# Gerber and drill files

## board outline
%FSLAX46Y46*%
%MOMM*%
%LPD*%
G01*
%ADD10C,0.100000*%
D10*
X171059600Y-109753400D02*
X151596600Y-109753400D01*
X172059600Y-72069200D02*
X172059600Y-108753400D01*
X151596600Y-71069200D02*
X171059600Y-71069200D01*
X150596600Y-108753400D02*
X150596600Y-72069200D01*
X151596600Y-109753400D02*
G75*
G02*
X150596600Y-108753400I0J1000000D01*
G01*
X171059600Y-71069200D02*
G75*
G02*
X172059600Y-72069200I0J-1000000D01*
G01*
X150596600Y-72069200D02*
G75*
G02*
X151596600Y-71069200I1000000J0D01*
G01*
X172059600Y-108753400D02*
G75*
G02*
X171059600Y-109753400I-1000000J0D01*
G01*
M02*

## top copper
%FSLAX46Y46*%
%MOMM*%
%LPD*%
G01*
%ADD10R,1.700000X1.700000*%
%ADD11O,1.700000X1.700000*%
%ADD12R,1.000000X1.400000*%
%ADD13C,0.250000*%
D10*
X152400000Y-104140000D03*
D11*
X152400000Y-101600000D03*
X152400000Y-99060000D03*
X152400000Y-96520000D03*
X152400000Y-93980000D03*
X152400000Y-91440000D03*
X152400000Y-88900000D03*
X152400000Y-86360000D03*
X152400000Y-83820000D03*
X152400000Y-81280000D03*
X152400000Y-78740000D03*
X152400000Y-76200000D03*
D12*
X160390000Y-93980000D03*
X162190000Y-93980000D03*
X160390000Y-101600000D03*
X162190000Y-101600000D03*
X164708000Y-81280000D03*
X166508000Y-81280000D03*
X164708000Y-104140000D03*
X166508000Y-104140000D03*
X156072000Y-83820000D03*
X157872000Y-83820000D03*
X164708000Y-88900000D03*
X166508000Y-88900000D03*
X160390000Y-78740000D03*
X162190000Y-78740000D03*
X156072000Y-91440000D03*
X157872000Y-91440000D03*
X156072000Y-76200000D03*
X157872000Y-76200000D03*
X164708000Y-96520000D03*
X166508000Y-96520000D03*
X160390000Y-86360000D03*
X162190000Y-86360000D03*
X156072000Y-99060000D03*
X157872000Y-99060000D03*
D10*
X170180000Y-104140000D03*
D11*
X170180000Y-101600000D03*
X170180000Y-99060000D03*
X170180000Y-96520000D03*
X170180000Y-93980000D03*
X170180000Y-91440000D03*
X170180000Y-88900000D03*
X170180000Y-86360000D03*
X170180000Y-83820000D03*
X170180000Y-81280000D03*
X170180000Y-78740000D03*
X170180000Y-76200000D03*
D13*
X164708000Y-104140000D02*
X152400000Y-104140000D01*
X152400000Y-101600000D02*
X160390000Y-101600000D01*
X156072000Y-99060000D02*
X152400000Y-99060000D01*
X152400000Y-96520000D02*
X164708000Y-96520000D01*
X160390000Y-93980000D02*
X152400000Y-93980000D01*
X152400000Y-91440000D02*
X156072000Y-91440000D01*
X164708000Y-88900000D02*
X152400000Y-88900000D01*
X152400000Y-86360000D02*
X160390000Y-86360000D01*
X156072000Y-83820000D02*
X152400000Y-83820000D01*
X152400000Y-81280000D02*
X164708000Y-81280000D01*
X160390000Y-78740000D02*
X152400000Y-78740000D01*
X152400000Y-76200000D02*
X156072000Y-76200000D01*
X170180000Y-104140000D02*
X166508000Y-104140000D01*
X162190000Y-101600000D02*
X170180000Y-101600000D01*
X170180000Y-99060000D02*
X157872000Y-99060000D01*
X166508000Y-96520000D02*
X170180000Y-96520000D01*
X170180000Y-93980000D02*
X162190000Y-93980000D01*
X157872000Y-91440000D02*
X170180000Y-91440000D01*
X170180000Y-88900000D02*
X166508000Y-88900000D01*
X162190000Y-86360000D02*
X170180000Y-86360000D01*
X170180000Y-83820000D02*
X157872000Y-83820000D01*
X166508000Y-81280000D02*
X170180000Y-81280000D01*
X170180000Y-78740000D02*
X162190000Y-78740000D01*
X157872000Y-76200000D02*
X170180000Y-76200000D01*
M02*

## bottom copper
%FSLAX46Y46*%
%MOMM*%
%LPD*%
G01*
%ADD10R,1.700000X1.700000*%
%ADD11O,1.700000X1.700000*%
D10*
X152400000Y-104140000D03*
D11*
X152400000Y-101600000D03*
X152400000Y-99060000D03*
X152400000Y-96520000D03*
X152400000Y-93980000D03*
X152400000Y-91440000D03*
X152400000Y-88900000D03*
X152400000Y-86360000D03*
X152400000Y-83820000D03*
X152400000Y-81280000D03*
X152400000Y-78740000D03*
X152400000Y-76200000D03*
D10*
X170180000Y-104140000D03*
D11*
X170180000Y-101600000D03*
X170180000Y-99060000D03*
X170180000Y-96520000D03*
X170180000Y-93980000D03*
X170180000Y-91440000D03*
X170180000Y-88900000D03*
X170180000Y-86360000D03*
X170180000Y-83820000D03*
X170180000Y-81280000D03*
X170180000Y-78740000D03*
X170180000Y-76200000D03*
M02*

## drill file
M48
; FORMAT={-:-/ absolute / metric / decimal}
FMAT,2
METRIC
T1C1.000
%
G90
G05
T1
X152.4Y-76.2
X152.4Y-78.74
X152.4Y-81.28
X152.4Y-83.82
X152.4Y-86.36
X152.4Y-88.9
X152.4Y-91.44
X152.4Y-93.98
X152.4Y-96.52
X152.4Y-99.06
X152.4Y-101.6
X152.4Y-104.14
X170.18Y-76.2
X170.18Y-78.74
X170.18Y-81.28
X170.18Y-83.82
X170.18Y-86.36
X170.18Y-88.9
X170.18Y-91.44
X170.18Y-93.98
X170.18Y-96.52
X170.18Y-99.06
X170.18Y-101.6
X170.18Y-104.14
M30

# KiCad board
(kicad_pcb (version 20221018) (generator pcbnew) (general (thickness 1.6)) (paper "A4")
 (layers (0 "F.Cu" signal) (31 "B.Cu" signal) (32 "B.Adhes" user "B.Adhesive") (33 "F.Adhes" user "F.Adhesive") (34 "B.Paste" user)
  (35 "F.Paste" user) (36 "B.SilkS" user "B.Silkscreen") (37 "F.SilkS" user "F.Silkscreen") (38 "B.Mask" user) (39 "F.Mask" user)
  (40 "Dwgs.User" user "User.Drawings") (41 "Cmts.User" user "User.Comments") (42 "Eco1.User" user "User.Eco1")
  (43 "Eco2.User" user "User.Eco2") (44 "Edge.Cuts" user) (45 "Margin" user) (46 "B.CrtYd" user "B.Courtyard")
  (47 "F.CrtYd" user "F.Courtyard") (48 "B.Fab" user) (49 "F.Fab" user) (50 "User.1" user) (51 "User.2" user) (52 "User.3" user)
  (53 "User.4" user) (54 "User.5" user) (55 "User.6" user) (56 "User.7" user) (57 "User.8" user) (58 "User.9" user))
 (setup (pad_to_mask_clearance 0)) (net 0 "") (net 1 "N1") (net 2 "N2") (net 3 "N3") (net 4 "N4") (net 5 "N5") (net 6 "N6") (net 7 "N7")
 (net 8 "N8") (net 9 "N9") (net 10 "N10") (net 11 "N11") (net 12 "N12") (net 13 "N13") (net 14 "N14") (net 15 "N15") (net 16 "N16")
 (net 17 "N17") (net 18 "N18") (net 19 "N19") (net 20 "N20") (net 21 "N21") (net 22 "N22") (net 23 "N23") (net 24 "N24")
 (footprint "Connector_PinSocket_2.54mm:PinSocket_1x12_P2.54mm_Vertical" (layer "F.Cu") (at 152.4 104.14 180)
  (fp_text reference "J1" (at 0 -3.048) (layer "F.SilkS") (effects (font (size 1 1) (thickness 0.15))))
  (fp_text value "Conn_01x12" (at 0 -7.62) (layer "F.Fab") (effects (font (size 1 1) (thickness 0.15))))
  (pad "1" thru_hole rect (at 0 0 180) (size 1.7 1.7) (drill 1) (layers "*.Cu" "*.Mask") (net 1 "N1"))
  (pad "2" thru_hole oval (at 0 2.54 180) (size 1.7 1.7) (drill 1) (layers "*.Cu" "*.Mask") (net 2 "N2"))
  (pad "3" thru_hole oval (at 0 5.08 180) (size 1.7 1.7) (drill 1) (layers "*.Cu" "*.Mask") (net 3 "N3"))
  (pad "4" thru_hole oval (at 0 7.62 180) (size 1.7 1.7) (drill 1) (layers "*.Cu" "*.Mask") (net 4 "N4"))
  (pad "5" thru_hole oval (at 0 10.16 180) (size 1.7 1.7) (drill 1) (layers "*.Cu" "*.Mask") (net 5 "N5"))
  (pad "6" thru_hole oval (at 0 12.7 180) (size 1.7 1.7) (drill 1) (layers "*.Cu" "*.Mask") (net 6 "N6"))
  (pad "7" thru_hole oval (at 0 15.24 180) (size 1.7 1.7) (drill 1) (layers "*.Cu" "*.Mask") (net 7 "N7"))
  (pad "8" thru_hole oval (at 0 17.78 180) (size 1.7 1.7) (drill 1) (layers "*.Cu" "*.Mask") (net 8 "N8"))
  (pad "9" thru_hole oval (at 0 20.32 180) (size 1.7 1.7) (drill 1) (layers "*.Cu" "*.Mask") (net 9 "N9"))
  (pad "10" thru_hole oval (at 0 22.86 180) (size 1.7 1.7) (drill 1) (layers "*.Cu" "*.Mask") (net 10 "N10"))
  (pad "11" thru_hole oval (at 0 25.4 180) (size 1.7 1.7) (drill 1) (layers "*.Cu" "*.Mask") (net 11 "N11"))
  (pad "12" thru_hole oval (at 0 27.94 180) (size 1.7 1.7) (drill 1) (layers "*.Cu" "*.Mask") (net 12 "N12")))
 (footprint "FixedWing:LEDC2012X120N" (layer "F.Cu") (at 161.29 93.98)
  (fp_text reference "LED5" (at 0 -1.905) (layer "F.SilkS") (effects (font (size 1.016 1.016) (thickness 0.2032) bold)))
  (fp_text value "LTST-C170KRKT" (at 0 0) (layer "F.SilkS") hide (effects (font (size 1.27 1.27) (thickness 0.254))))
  (pad "1" smd rect (at -0.9 0) (size 1 1.4) (layers "F.Cu" "F.Paste" "F.Mask") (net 5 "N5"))
  (pad "2" smd rect (at 0.9 0) (size 1 1.4) (layers "F.Cu" "F.Paste" "F.Mask") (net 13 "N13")))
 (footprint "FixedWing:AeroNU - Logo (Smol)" (layer "F.Cu") (at 157.380649 109.377388)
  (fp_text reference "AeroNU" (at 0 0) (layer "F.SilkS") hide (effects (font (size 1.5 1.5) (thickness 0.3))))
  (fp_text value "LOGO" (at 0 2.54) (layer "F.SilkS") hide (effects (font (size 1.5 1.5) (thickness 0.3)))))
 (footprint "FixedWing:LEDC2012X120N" (layer "F.Cu") (at 161.29 101.6)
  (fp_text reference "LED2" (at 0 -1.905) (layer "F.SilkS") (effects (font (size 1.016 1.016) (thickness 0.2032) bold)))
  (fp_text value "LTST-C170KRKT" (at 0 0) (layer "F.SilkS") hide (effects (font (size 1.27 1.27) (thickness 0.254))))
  (pad "1" smd rect (at -0.9 0) (size 1 1.4) (layers "F.Cu" "F.Paste" "F.Mask") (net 2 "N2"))
  (pad "2" smd rect (at 0.9 0) (size 1 1.4) (layers "F.Cu" "F.Paste" "F.Mask") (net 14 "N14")))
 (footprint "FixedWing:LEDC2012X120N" (layer "F.Cu") (at 165.608 81.28)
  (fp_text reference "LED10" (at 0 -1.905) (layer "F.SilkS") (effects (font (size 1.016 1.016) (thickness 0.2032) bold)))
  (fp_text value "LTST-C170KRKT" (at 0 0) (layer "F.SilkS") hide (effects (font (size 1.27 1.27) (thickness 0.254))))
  (pad "1" smd rect (at -0.9 0) (size 1 1.4) (layers "F.Cu" "F.Paste" "F.Mask") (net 10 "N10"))
  (pad "2" smd rect (at 0.9 0) (size 1 1.4) (layers "F.Cu" "F.Paste" "F.Mask") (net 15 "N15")))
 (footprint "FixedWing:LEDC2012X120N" (layer "F.Cu") (at 165.608 104.14)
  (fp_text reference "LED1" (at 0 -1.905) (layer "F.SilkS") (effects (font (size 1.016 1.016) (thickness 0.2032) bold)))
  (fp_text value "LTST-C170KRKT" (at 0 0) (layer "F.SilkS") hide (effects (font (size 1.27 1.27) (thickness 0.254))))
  (pad "1" smd rect (at -0.9 0) (size 1 1.4) (layers "F.Cu" "F.Paste" "F.Mask") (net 1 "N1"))
  (pad "2" smd rect (at 0.9 0) (size 1 1.4) (layers "F.Cu" "F.Paste" "F.Mask") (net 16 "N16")))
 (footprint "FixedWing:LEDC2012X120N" (layer "F.Cu") (at 156.972 83.82)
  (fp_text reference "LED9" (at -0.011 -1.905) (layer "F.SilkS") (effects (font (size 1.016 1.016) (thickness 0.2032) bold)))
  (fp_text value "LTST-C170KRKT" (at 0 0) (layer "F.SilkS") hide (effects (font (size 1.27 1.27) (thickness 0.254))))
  (pad "1" smd rect (at -0.9 0) (size 1 1.4) (layers "F.Cu" "F.Paste" "F.Mask") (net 9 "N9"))
  (pad "2" smd rect (at 0.9 0) (size 1 1.4) (layers "F.Cu" "F.Paste" "F.Mask") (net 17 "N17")))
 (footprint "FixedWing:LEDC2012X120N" (layer "F.Cu") (at 165.608 88.9)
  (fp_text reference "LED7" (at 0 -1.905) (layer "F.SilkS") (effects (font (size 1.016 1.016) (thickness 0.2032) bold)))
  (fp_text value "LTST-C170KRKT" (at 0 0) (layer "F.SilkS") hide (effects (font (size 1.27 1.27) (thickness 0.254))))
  (pad "1" smd rect (at -0.9 0) (size 1 1.4) (layers "F.Cu" "F.Paste" "F.Mask") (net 7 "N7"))
  (pad "2" smd rect (at 0.9 0) (size 1 1.4) (layers "F.Cu" "F.Paste" "F.Mask") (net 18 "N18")))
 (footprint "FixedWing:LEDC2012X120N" (layer "F.Cu") (at 161.29 78.74)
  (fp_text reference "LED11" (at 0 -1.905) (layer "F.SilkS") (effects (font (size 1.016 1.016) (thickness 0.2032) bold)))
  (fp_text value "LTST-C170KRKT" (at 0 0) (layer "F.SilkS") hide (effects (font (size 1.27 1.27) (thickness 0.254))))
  (pad "1" smd rect (at -0.9 0) (size 1 1.4) (layers "F.Cu" "F.Paste" "F.Mask") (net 11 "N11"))
  (pad "2" smd rect (at 0.9 0) (size 1 1.4) (layers "F.Cu" "F.Paste" "F.Mask") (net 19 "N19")))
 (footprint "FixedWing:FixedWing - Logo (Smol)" (layer "F.Cu") (at 165.3921 73.1774)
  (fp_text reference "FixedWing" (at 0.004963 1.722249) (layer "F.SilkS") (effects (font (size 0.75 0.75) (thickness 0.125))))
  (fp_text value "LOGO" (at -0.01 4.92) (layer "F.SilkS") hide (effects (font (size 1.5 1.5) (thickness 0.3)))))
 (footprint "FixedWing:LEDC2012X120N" (layer "F.Cu") (at 156.972 91.44)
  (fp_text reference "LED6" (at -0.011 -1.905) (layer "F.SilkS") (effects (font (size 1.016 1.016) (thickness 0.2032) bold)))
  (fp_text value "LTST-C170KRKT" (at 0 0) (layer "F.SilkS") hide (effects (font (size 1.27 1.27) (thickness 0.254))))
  (pad "1" smd rect (at -0.9 0) (size 1 1.4) (layers "F.Cu" "F.Paste" "F.Mask") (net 6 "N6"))
  (pad "2" smd rect (at 0.9 0) (size 1 1.4) (layers "F.Cu" "F.Paste" "F.Mask") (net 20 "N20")))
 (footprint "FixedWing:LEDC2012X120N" (layer "F.Cu") (at 156.972 76.2)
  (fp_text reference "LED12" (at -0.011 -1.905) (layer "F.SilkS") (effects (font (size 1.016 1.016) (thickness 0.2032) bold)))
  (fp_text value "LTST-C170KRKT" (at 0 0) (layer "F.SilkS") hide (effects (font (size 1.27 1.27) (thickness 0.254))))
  (pad "1" smd rect (at -0.9 0) (size 1 1.4) (layers "F.Cu" "F.Paste" "F.Mask") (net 12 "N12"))
  (pad "2" smd rect (at 0.9 0) (size 1 1.4) (layers "F.Cu" "F.Paste" "F.Mask") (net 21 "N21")))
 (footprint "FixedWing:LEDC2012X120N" (layer "F.Cu") (at 165.608 96.52)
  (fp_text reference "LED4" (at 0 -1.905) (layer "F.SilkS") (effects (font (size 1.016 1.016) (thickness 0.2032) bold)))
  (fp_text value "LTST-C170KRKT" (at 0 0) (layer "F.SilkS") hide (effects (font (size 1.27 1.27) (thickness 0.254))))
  (pad "1" smd rect (at -0.9 0) (size 1 1.4) (layers "F.Cu" "F.Paste" "F.Mask") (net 4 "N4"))
  (pad "2" smd rect (at 0.9 0) (size 1 1.4) (layers "F.Cu" "F.Paste" "F.Mask") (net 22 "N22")))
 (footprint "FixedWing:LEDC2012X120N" (layer "F.Cu") (at 161.29 86.36)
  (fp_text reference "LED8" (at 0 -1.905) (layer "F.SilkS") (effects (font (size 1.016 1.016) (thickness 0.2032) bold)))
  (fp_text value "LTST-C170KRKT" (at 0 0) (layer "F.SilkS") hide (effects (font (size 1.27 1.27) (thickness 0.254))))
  (pad "1" smd rect (at -0.9 0) (size 1 1.4) (layers "F.Cu" "F.Paste" "F.Mask") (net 8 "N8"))
  (pad "2" smd rect (at 0.9 0) (size 1 1.4) (layers "F.Cu" "F.Paste" "F.Mask") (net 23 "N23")))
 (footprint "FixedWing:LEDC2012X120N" (layer "F.Cu") (at 156.972 99.06)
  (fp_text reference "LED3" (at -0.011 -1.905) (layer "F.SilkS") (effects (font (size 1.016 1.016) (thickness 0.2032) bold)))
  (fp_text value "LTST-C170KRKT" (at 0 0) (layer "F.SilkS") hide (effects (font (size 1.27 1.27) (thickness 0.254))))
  (pad "1" smd rect (at -0.9 0) (size 1 1.4) (layers "F.Cu" "F.Paste" "F.Mask") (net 3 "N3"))
  (pad "2" smd rect (at 0.9 0) (size 1 1.4) (layers "F.Cu" "F.Paste" "F.Mask") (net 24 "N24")))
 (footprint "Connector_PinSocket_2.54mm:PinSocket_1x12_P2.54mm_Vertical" (layer "F.Cu") (at 170.18 104.14 180)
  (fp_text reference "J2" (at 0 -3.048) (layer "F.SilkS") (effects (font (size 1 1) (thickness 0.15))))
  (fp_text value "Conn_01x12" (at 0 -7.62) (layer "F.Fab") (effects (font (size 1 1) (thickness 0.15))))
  (pad "1" thru_hole rect (at 0 0 180) (size 1.7 1.7) (drill 1) (layers "*.Cu" "*.Mask") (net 16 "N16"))
  (pad "2" thru_hole oval (at 0 2.54 180) (size 1.7 1.7) (drill 1) (layers "*.Cu" "*.Mask") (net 14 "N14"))
  (pad "3" thru_hole oval (at 0 5.08 180) (size 1.7 1.7) (drill 1) (layers "*.Cu" "*.Mask") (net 24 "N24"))
  (pad "4" thru_hole oval (at 0 7.62 180) (size 1.7 1.7) (drill 1) (layers "*.Cu" "*.Mask") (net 22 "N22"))
  (pad "5" thru_hole oval (at 0 10.16 180) (size 1.7 1.7) (drill 1) (layers "*.Cu" "*.Mask") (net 13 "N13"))
  (pad "6" thru_hole oval (at 0 12.7 180) (size 1.7 1.7) (drill 1) (layers "*.Cu" "*.Mask") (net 20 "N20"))
  (pad "7" thru_hole oval (at 0 15.24 180) (size 1.7 1.7) (drill 1) (layers "*.Cu" "*.Mask") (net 18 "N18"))
  (pad "8" thru_hole oval (at 0 17.78 180) (size 1.7 1.7) (drill 1) (layers "*.Cu" "*.Mask") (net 23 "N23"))
  (pad "9" thru_hole oval (at 0 20.32 180) (size 1.7 1.7) (drill 1) (layers "*.Cu" "*.Mask") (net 17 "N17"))
  (pad "10" thru_hole oval (at 0 22.86 180) (size 1.7 1.7) (drill 1) (layers "*.Cu" "*.Mask") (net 15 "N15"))
  (pad "11" thru_hole oval (at 0 25.4 180) (size 1.7 1.7) (drill 1) (layers "*.Cu" "*.Mask") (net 19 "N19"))
  (pad "12" thru_hole oval (at 0 27.94 180) (size 1.7 1.7) (drill 1) (layers "*.Cu" "*.Mask") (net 21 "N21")))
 (gr_line (start 171.0596 109.7534) (end 151.5966 109.7534) (stroke (width 0.1) (type default)) (layer "Edge.Cuts"))
 (gr_line (start 172.0596 72.0692) (end 172.0596 108.7534) (stroke (width 0.1) (type default)) (layer "Edge.Cuts"))
 (gr_line (start 151.5966 71.0692) (end 171.0596 71.0692) (stroke (width 0.1) (type default)) (layer "Edge.Cuts"))
 (gr_line (start 150.5966 108.7534) (end 150.5966 72.0692) (stroke (width 0.1) (type default)) (layer "Edge.Cuts"))
 (gr_arc (start 151.5966 109.7534) (mid 150.889493 109.460507) (end 150.5966 108.7534) (stroke (width 0.1) (type default))
  (layer "Edge.Cuts"))
 (gr_arc (start 171.0596 71.0692) (mid 171.766707 71.362093) (end 172.0596 72.0692) (stroke (width 0.1) (type default)) (layer "Edge.Cuts"))
 (gr_arc (start 150.5966 72.0692) (mid 150.889493 71.362093) (end 151.5966 71.0692) (stroke (width 0.1) (type default)) (layer "Edge.Cuts"))
 (gr_arc (start 172.0596 108.7534) (mid 171.766707 109.460507) (end 171.0596 109.7534) (stroke (width 0.1) (type default))
  (layer "Edge.Cuts"))
 (segment (start 164.708 104.14) (end 152.4 104.14) (width 0.25) (layer "F.Cu") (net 1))
 (segment (start 152.4 101.6) (end 160.39 101.6) (width 0.25) (layer "F.Cu") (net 2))
 (segment (start 156.072 99.06) (end 152.4 99.06) (width 0.25) (layer "F.Cu") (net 3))
 (segment (start 152.4 96.52) (end 164.708 96.52) (width 0.25) (layer "F.Cu") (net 4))
 (segment (start 160.39 93.98) (end 152.4 93.98) (width 0.25) (layer "F.Cu") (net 5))
 (segment (start 152.4 91.44) (end 156.072 91.44) (width 0.25) (layer "F.Cu") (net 6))
 (segment (start 164.708 88.9) (end 152.4 88.9) (width 0.25) (layer "F.Cu") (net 7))
 (segment (start 152.4 86.36) (end 160.39 86.36) (width 0.25) (layer "F.Cu") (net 8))
 (segment (start 156.072 83.82) (end 152.4 83.82) (width 0.25) (layer "F.Cu") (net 9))
 (segment (start 152.4 81.28) (end 164.708 81.28) (width 0.25) (layer "F.Cu") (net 10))
 (segment (start 160.39 78.74) (end 152.4 78.74) (width 0.25) (layer "F.Cu") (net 11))
 (segment (start 152.4 76.2) (end 156.072 76.2) (width 0.25) (layer "F.Cu") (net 12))
 (segment (start 170.18 104.14) (end 166.508 104.14) (width 0.25) (layer "F.Cu") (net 16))
 (segment (start 162.19 101.6) (end 170.18 101.6) (width 0.25) (layer "F.Cu") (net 14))
 (segment (start 170.18 99.06) (end 157.872 99.06) (width 0.25) (layer "F.Cu") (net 24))
 (segment (start 166.508 96.52) (end 170.18 96.52) (width 0.25) (layer "F.Cu") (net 22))
 (segment (start 170.18 93.98) (end 162.19 93.98) (width 0.25) (layer "F.Cu") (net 13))
 (segment (start 157.872 91.44) (end 170.18 91.44) (width 0.25) (layer "F.Cu") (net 20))
 (segment (start 170.18 88.9) (end 166.508 88.9) (width 0.25) (layer "F.Cu") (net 18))
 (segment (start 162.19 86.36) (end 170.18 86.36) (width 0.25) (layer "F.Cu") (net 23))
 (segment (start 170.18 83.82) (end 157.872 83.82) (width 0.25) (layer "F.Cu") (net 17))
 (segment (start 166.508 81.28) (end 170.18 81.28) (width 0.25) (layer "F.Cu") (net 15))
 (segment (start 170.18 78.74) (end 162.19 78.74) (width 0.25) (layer "F.Cu") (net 19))
 (segment (start 157.872 76.2) (end 170.18 76.2) (width 0.25) (layer "F.Cu") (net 21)))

